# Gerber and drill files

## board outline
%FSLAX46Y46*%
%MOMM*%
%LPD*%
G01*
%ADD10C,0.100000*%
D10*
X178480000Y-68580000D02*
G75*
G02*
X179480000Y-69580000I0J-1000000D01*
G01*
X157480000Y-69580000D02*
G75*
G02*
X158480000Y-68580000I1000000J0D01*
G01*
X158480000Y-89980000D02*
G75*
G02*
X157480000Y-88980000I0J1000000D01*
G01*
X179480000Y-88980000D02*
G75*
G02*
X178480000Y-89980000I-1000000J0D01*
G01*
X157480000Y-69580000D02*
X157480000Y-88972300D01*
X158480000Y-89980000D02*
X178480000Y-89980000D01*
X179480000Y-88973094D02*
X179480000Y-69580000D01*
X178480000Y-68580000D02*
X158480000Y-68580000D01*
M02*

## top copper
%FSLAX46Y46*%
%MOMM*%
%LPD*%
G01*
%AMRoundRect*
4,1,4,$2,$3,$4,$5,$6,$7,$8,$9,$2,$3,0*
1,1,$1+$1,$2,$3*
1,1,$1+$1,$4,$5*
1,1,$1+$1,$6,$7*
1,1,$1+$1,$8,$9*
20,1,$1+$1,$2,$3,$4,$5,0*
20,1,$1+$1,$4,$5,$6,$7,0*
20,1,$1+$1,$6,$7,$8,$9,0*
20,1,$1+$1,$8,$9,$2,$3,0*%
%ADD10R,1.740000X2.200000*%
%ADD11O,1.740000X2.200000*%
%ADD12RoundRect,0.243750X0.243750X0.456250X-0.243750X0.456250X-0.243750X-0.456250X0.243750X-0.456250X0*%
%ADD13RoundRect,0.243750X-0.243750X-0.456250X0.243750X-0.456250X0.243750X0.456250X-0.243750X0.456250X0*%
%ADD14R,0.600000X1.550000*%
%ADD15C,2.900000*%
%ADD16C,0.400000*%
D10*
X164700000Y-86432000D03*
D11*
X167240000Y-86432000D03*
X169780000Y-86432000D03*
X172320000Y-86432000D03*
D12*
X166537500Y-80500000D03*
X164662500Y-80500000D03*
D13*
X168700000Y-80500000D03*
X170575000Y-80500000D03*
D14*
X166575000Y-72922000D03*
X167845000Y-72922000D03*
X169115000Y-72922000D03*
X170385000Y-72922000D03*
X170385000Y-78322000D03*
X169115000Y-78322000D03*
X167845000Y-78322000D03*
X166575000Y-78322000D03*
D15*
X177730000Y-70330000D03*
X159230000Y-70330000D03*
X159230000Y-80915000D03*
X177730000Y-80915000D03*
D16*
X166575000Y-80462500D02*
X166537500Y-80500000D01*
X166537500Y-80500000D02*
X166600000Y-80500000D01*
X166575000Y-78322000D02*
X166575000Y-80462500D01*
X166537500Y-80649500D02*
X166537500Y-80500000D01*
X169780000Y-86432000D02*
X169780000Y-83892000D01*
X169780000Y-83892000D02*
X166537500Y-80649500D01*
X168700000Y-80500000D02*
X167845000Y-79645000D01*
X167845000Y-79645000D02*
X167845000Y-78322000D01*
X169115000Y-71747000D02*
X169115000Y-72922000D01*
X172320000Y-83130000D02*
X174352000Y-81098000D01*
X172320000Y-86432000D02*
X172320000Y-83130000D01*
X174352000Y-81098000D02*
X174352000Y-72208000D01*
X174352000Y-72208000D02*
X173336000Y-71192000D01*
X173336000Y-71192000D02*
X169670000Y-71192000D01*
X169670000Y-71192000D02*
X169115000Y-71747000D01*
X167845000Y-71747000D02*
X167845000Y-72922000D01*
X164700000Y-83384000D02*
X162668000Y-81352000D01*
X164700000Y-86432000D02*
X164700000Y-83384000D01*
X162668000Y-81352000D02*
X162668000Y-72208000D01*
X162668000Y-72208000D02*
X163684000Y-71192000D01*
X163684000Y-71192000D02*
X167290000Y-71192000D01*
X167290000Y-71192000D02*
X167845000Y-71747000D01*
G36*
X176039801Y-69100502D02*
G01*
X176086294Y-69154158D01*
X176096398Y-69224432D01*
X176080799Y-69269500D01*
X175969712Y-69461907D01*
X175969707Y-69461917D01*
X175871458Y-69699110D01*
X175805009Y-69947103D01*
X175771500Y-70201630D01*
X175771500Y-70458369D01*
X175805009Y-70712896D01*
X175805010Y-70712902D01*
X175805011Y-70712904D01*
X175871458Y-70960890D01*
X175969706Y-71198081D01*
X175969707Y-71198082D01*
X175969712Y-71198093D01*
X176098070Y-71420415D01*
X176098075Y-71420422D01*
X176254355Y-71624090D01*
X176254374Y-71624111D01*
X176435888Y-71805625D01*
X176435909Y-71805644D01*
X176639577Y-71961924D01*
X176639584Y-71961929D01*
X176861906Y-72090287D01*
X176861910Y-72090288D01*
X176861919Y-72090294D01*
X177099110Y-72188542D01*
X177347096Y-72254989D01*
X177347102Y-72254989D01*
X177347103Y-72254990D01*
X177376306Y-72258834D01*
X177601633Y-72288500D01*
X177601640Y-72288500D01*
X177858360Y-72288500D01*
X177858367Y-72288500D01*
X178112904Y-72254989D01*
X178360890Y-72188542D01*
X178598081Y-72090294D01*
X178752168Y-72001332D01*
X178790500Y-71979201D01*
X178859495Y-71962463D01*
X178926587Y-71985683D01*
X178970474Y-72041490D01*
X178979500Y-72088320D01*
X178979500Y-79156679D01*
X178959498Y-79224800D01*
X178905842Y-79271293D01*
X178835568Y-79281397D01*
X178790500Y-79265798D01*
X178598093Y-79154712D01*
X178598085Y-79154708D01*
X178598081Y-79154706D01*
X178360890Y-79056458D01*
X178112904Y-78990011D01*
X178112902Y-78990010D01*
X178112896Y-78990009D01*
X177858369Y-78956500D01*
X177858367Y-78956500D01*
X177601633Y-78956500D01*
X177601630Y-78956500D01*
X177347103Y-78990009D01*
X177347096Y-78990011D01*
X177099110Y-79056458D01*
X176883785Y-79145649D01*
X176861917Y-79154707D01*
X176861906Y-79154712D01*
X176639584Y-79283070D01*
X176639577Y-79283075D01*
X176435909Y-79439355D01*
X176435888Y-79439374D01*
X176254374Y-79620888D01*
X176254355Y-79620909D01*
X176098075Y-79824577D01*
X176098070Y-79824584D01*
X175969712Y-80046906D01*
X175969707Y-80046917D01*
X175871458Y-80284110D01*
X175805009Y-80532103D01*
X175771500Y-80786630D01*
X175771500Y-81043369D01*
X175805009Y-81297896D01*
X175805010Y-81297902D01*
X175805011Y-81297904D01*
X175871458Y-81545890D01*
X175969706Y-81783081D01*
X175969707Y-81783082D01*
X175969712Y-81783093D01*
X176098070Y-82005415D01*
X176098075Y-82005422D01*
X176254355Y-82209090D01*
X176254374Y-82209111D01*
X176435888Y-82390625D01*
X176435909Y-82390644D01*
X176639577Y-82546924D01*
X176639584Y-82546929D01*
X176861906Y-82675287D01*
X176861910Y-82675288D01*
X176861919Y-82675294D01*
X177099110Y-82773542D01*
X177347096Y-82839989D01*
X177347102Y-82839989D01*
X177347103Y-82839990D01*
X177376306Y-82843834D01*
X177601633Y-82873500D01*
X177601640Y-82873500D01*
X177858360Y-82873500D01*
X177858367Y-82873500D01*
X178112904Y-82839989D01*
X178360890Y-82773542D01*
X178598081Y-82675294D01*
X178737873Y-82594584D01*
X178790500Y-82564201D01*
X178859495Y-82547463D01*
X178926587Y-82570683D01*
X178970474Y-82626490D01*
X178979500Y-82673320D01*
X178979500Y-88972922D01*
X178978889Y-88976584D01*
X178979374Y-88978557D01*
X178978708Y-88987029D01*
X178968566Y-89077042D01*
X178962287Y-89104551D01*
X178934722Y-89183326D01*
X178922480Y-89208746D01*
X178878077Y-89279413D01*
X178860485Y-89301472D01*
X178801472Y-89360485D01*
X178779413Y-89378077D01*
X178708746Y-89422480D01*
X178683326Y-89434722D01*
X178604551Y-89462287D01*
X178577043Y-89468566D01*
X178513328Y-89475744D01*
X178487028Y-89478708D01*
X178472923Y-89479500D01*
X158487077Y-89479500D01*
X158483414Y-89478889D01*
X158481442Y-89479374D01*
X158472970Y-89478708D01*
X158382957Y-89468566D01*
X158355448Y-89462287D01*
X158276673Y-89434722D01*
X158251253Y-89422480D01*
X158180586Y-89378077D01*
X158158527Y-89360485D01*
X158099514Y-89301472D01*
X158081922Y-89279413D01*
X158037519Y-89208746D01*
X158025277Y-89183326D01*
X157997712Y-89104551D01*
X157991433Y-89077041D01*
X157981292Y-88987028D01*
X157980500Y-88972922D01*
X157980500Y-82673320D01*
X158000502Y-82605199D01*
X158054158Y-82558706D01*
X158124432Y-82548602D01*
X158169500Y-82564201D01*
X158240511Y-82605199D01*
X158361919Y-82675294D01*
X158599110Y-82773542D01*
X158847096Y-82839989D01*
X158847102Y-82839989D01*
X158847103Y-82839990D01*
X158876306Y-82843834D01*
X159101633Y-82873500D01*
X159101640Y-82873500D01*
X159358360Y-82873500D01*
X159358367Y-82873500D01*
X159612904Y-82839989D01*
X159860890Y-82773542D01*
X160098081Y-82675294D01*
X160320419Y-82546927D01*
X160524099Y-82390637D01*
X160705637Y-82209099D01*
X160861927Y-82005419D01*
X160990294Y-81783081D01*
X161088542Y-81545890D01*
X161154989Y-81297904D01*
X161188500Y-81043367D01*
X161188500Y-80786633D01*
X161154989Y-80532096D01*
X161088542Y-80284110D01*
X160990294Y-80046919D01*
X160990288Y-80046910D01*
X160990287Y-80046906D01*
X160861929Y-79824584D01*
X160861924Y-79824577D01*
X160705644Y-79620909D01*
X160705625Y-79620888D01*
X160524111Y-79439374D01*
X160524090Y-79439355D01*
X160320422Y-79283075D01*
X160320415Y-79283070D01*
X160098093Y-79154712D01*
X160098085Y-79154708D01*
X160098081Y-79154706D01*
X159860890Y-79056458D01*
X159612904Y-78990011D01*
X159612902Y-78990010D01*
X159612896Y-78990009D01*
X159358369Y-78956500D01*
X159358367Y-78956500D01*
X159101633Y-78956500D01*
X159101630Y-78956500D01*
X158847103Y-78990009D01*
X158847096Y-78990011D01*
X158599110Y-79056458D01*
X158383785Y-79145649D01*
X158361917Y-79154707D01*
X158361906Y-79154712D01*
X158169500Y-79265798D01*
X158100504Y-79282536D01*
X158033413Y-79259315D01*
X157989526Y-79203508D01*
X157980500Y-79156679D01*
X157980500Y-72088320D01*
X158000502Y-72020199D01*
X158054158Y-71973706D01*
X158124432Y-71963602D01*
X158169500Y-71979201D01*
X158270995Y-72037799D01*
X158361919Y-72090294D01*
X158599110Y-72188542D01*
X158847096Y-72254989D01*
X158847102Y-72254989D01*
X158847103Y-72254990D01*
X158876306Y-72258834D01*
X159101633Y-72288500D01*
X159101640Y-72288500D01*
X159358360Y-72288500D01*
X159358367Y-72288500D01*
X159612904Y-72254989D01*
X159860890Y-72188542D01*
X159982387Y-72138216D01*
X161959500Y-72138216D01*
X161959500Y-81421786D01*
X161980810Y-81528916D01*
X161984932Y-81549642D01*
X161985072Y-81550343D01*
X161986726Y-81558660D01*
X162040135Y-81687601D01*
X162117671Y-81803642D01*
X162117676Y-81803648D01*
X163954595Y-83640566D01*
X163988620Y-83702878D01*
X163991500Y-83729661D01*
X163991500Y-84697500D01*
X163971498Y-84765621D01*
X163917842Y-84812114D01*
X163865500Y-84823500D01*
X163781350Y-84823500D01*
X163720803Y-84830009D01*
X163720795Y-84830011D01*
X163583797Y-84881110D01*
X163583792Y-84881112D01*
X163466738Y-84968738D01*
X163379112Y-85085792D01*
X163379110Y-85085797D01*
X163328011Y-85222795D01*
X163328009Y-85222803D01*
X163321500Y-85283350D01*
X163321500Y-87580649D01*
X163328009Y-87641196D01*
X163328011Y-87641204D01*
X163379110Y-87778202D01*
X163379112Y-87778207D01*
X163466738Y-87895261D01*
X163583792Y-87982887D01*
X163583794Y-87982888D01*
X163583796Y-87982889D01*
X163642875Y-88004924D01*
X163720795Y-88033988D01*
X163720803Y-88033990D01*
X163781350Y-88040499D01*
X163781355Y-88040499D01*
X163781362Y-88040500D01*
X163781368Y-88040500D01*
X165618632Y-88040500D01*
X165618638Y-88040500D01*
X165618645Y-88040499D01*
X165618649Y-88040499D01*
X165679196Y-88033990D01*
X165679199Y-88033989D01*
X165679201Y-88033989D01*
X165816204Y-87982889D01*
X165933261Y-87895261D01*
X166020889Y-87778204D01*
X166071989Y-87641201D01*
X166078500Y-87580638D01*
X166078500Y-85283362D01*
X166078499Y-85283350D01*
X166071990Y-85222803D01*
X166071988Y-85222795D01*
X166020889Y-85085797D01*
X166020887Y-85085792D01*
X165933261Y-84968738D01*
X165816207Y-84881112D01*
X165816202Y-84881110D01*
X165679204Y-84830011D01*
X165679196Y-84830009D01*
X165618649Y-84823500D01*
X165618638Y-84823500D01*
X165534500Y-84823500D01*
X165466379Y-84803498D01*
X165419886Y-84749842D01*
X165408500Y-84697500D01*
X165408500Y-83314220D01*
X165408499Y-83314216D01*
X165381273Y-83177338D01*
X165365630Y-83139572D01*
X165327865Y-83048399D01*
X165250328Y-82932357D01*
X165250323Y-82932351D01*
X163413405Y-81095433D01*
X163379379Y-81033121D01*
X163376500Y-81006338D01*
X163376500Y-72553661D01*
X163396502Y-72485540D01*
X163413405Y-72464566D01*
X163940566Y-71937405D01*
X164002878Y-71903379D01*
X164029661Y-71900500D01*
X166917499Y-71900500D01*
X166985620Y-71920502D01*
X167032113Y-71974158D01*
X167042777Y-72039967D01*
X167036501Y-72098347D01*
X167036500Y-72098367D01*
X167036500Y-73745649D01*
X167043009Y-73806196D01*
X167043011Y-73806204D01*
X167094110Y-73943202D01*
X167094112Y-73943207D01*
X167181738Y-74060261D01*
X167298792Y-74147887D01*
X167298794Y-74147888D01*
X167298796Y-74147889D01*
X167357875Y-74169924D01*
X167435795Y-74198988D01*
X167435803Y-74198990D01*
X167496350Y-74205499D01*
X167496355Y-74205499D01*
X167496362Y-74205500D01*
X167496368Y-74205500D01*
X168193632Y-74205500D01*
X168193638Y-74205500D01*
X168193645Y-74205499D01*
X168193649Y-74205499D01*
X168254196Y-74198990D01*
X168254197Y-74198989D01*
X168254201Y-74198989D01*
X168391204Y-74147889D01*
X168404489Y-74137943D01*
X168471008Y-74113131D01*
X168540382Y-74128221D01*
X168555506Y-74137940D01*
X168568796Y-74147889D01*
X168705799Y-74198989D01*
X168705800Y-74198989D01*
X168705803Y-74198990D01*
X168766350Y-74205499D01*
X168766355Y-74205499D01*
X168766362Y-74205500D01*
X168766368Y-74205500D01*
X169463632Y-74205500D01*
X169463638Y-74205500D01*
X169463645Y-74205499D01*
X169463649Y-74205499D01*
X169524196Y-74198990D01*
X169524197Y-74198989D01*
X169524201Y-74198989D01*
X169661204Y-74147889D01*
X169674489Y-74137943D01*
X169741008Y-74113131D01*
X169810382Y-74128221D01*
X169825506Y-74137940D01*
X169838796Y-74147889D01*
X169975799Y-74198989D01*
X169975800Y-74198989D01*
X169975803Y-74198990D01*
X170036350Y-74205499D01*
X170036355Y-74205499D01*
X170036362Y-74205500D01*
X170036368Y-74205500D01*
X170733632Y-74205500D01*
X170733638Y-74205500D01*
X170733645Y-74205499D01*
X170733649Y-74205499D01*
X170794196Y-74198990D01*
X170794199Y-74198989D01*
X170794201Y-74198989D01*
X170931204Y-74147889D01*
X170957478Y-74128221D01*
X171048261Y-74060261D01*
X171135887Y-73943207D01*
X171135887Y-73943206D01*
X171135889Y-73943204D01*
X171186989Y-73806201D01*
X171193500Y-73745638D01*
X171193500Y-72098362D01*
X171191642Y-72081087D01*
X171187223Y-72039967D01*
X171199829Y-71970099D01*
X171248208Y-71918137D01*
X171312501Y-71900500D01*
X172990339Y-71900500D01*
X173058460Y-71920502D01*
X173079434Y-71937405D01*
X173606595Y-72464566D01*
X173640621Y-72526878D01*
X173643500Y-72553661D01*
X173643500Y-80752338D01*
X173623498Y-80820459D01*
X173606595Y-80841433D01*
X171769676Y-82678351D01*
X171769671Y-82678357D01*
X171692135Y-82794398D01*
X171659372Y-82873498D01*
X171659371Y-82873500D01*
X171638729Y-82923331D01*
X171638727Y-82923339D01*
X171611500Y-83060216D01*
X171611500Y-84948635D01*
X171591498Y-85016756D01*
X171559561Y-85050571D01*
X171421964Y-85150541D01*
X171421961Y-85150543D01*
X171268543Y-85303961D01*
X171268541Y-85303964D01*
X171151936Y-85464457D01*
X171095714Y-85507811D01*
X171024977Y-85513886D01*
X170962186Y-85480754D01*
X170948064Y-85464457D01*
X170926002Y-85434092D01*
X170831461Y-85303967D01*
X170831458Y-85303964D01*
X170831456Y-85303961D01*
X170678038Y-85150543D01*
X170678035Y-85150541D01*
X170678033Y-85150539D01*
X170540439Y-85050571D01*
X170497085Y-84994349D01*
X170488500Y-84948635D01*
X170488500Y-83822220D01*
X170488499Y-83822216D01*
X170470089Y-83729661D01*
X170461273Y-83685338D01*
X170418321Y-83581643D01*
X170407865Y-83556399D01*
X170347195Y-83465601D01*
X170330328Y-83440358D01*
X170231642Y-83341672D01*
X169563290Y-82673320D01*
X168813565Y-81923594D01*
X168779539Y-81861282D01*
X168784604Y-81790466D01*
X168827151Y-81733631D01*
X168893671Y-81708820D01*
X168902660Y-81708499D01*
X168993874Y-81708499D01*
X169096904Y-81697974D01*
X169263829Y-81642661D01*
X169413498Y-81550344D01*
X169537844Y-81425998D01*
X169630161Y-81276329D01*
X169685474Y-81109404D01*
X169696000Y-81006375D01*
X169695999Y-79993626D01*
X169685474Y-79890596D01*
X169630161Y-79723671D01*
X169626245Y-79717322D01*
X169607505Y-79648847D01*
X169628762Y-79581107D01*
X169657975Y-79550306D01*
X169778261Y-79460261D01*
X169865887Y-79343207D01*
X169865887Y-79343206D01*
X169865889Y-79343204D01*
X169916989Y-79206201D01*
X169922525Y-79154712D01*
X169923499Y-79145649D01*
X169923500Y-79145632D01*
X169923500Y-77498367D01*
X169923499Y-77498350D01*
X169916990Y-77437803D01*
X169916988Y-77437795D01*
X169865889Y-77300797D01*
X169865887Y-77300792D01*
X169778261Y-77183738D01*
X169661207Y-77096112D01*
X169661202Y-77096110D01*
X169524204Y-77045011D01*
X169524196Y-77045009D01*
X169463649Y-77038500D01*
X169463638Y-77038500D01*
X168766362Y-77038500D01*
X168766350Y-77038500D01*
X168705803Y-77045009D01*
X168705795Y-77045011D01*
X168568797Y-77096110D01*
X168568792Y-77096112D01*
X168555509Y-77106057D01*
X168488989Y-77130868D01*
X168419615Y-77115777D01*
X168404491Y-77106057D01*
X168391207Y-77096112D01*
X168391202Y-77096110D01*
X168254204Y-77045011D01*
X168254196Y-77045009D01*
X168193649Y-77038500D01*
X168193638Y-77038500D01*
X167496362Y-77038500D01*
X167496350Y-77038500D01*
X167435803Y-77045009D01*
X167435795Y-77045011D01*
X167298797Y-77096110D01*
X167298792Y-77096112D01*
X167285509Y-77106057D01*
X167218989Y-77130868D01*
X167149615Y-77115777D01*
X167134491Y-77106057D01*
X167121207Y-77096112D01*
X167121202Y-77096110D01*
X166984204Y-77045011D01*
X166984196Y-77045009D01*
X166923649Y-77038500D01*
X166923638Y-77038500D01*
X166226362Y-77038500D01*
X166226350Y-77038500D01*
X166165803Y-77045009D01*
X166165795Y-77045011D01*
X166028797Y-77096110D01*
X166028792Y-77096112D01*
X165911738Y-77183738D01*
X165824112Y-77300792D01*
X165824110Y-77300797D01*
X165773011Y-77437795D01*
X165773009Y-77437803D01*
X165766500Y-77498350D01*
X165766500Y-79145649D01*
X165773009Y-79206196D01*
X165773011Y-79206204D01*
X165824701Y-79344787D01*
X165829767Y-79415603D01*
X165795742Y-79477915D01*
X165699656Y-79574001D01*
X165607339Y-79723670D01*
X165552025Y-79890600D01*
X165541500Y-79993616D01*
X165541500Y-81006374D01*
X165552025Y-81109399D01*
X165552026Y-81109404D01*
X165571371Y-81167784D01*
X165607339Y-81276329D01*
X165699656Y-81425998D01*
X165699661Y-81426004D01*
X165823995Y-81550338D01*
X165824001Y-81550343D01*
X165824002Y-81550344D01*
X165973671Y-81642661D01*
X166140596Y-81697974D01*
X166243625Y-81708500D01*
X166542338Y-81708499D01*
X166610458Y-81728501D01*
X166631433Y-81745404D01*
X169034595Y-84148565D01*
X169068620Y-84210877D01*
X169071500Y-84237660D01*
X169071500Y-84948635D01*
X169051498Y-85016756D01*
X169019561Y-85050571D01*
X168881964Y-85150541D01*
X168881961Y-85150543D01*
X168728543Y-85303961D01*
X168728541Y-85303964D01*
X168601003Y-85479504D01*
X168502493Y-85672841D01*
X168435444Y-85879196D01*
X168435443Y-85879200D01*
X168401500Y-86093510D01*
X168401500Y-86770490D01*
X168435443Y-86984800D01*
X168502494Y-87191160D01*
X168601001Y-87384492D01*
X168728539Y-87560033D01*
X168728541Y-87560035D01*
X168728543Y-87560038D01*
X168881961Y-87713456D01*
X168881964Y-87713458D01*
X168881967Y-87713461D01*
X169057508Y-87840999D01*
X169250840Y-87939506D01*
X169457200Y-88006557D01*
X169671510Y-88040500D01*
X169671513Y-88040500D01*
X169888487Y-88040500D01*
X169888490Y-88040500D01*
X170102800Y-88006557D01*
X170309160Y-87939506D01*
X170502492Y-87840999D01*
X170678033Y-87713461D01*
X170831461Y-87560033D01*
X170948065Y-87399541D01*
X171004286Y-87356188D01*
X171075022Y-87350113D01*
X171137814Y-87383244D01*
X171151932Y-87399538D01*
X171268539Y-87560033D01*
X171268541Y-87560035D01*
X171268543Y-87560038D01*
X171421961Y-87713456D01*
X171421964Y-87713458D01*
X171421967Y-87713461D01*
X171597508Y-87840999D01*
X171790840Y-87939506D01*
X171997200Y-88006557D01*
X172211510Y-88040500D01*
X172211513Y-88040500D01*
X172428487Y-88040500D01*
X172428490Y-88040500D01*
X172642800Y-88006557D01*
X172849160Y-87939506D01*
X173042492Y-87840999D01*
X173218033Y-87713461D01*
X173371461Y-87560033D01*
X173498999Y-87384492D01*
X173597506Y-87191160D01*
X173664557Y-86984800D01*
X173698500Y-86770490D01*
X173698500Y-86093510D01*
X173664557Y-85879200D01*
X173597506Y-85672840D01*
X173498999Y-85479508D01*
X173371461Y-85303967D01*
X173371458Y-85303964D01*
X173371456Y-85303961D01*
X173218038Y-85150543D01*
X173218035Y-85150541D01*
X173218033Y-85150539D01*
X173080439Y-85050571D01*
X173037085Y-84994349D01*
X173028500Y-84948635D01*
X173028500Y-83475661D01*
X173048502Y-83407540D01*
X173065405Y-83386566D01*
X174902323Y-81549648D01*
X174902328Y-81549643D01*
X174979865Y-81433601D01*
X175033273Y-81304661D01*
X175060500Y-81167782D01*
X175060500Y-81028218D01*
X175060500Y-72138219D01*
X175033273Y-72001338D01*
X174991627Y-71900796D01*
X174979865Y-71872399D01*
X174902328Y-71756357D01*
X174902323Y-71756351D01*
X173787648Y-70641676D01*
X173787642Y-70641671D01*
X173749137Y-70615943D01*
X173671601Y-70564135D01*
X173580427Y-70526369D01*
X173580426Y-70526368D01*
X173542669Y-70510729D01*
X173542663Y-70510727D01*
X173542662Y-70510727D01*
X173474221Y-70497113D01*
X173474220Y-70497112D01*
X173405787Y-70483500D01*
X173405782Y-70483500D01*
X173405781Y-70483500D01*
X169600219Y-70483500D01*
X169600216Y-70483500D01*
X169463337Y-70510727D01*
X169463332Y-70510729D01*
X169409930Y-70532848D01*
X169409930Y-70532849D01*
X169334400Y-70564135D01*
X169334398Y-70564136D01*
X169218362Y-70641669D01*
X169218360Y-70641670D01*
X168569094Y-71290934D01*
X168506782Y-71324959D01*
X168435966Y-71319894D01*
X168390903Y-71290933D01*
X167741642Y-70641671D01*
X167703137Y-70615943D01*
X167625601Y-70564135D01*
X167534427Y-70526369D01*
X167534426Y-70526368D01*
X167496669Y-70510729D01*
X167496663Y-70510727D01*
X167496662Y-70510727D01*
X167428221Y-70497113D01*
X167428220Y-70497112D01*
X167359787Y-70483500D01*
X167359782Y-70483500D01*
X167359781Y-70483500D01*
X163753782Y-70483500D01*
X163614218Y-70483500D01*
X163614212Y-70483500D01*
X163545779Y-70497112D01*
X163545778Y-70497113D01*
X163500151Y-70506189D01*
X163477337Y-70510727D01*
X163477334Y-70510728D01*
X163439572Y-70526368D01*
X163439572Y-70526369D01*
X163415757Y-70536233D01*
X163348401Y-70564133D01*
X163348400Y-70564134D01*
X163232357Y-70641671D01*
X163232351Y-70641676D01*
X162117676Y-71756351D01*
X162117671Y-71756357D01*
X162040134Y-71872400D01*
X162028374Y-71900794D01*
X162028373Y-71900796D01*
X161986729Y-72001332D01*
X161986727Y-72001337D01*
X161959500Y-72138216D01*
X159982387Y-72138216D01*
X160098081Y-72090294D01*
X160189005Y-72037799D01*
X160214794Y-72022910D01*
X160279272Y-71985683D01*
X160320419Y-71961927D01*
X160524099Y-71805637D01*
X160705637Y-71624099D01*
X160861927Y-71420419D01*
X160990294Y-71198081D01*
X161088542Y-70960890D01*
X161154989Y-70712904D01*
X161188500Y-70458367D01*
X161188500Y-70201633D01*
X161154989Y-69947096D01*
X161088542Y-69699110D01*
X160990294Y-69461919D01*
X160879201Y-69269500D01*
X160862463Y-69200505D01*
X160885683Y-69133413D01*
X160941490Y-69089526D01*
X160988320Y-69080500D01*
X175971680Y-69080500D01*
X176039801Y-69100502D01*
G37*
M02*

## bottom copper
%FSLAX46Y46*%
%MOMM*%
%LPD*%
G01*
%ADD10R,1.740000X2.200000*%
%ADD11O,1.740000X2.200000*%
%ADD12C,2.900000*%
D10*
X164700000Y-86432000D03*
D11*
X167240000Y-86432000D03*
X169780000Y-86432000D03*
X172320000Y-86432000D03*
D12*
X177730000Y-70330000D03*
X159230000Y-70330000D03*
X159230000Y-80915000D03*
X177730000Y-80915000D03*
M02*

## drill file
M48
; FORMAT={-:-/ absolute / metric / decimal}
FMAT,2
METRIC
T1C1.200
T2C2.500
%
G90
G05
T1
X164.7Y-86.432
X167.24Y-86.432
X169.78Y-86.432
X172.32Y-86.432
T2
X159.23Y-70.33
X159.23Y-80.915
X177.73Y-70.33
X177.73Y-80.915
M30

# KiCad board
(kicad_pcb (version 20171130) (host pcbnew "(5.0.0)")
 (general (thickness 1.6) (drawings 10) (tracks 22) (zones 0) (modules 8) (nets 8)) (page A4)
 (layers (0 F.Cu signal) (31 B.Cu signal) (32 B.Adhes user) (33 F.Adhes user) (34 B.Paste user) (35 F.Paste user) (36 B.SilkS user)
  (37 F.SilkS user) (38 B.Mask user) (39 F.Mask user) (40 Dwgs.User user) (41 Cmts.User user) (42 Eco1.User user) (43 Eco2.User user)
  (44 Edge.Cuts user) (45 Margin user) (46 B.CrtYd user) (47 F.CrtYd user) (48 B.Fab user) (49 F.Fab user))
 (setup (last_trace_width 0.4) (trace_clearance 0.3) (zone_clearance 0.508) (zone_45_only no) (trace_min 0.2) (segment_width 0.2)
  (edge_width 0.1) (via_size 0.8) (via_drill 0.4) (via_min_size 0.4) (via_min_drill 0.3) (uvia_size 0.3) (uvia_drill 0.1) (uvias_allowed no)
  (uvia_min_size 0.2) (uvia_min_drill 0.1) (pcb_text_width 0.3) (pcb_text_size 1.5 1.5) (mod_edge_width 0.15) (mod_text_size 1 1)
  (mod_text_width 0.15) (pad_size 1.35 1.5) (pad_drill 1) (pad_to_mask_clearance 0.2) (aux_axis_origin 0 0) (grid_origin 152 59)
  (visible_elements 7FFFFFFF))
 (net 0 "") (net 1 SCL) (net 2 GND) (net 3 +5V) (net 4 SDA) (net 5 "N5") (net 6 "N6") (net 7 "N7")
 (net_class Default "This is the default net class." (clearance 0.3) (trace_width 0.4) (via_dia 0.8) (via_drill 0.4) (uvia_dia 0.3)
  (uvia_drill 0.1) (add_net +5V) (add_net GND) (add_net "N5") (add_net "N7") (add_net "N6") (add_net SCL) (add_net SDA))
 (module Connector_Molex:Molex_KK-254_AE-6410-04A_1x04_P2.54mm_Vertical (layer F.Cu) (at 164.7 86.432)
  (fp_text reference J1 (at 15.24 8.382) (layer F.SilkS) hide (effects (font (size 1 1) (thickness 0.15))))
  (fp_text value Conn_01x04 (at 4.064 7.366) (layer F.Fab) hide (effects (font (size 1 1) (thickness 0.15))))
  (pad 1 thru_hole rect (at 0 0) (size 1.74 2.2) (drill 1.2) (layers *.Cu *.Mask) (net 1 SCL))
  (pad 2 thru_hole oval (at 2.54 0) (size 1.74 2.2) (drill 1.2) (layers *.Cu *.Mask) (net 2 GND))
  (pad 3 thru_hole oval (at 5.08 0) (size 1.74 2.2) (drill 1.2) (layers *.Cu *.Mask) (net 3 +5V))
  (pad 4 thru_hole oval (at 7.62 0) (size 1.74 2.2) (drill 1.2) (layers *.Cu *.Mask) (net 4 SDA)))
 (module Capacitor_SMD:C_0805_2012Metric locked (layer F.Cu) (at 165.6 80.5 180)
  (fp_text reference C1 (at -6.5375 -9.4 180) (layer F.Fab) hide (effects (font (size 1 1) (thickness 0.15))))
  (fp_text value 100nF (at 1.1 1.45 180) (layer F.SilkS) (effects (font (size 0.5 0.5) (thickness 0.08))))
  (pad 1 smd roundrect (at -0.9375 0 180) (size 0.975 1.4) (layers F.Cu F.Paste F.Mask) (roundrect_rratio 0.25) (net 3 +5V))
  (pad 2 smd roundrect (at 0.9375 0 180) (size 0.975 1.4) (layers F.Cu F.Paste F.Mask) (roundrect_rratio 0.25) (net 2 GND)))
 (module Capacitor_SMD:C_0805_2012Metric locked (layer F.Cu) (at 169.6375 80.5)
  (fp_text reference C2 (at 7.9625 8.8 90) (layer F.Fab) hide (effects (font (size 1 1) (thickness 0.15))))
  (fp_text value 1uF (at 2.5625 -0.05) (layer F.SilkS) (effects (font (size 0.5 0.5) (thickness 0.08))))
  (pad 1 smd roundrect (at -0.9375 0) (size 0.975 1.4) (layers F.Cu F.Paste F.Mask) (roundrect_rratio 0.25) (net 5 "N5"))
  (pad 2 smd roundrect (at 0.9375 0) (size 0.975 1.4) (layers F.Cu F.Paste F.Mask) (roundrect_rratio 0.25) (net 2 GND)))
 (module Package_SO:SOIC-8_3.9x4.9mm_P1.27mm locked (layer F.Cu) (at 168.48 75.622 90)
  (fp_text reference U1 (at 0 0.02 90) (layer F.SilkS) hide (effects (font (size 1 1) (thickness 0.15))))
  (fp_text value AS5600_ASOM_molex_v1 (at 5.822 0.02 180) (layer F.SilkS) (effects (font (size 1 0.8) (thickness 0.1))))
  (pad 8 smd rect (at 2.7 -1.905 90) (size 1.55 0.6) (layers F.Cu F.Paste F.Mask) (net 2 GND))
  (pad 7 smd rect (at 2.7 -0.635 90) (size 1.55 0.6) (layers F.Cu F.Paste F.Mask) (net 1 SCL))
  (pad 6 smd rect (at 2.7 0.635 90) (size 1.55 0.6) (layers F.Cu F.Paste F.Mask) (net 4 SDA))
  (pad 5 smd rect (at 2.7 1.905 90) (size 1.55 0.6) (layers F.Cu F.Paste F.Mask) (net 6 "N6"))
  (pad 4 smd rect (at -2.7 1.905 90) (size 1.55 0.6) (layers F.Cu F.Paste F.Mask) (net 2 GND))
  (pad 3 smd rect (at -2.7 0.635 90) (size 1.55 0.6) (layers F.Cu F.Paste F.Mask) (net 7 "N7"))
  (pad 2 smd rect (at -2.7 -0.635 90) (size 1.55 0.6) (layers F.Cu F.Paste F.Mask) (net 5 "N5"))
  (pad 1 smd rect (at -2.7 -1.905 90) (size 1.55 0.6) (layers F.Cu F.Paste F.Mask) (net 3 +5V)))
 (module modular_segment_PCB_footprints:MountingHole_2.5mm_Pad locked (layer F.Cu) (at 177.73 70.33)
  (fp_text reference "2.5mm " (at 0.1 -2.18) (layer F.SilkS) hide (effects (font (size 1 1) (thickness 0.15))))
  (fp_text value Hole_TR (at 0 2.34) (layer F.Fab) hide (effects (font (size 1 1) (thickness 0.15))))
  (pad "" np_thru_hole circle (at 0 0) (size 2.9 2.9) (drill 2.5) (layers *.Cu *.Mask)))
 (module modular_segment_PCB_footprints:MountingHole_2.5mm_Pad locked (layer F.Cu) (at 159.23 70.33)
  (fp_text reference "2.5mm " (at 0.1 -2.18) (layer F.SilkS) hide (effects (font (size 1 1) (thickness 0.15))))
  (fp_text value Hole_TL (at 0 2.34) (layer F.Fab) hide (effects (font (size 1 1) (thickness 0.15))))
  (pad "" np_thru_hole circle (at 0 0) (size 2.9 2.9) (drill 2.5) (layers *.Cu *.Mask)))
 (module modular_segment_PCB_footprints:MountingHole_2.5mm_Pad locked (layer F.Cu) (at 159.23 80.915)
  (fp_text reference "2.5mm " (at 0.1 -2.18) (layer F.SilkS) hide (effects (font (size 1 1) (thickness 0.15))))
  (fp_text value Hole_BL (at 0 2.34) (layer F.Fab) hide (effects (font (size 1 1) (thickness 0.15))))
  (pad "" np_thru_hole circle (at 0 0) (size 2.9 2.9) (drill 2.5) (layers *.Cu *.Mask)))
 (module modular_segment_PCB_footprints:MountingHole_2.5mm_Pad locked (layer F.Cu) (at 177.73 80.915)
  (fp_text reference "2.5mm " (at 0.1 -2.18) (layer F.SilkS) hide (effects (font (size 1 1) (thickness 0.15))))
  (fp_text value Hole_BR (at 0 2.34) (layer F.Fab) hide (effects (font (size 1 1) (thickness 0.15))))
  (pad "" np_thru_hole circle (at 0 0) (size 2.9 2.9) (drill 2.5) (layers *.Cu *.Mask)))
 (gr_arc (start 178.48 69.58) (end 179.48 69.58) (angle -90) (layer Edge.Cuts) (width 0.1))
 (gr_arc (start 158.48 69.58) (end 158.48 68.58) (angle -90) (layer Edge.Cuts) (width 0.1))
 (gr_arc (start 158.48 88.98) (end 157.48 88.98) (angle -90) (layer Edge.Cuts) (width 0.1))
 (gr_arc (start 178.48 88.98) (end 178.48 89.98) (angle -90) (layer Edge.Cuts) (width 0.1))
 (gr_line (start 157.48 69.58) (end 157.48 88.9723) (layer Edge.Cuts) (width 0.1))
 (gr_line (start 158.48 89.98) (end 178.48 89.98) (layer Edge.Cuts) (width 0.1))
 (gr_line (start 179.48 88.973094) (end 179.48 69.58) (layer Edge.Cuts) (width 0.1))
 (gr_line (start 178.48 68.58) (end 158.48 68.58) (layer Edge.Cuts) (width 0.1))
 (segment (start 166.575 80.4625) (end 166.5375 80.5) (width 0.4) (layer F.Cu) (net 3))
 (segment (start 166.5375 80.5) (end 166.6 80.5) (width 0.4) (layer F.Cu) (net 3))
 (segment (start 166.575 78.322) (end 166.575 80.4625) (width 0.4) (layer F.Cu) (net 3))
 (segment (start 166.5375 80.6495) (end 166.5375 80.5) (width 0.4) (layer F.Cu) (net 3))
 (segment (start 169.78 86.432) (end 169.78 83.892) (width 0.4) (layer F.Cu) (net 3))
 (segment (start 169.78 83.892) (end 166.5375 80.6495) (width 0.4) (layer F.Cu) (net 3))
 (segment (start 168.7 80.5) (end 167.845 79.645) (width 0.4) (layer F.Cu) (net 5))
 (segment (start 167.845 79.645) (end 167.845 78.322) (width 0.4) (layer F.Cu) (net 5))
 (segment (start 169.115 71.747) (end 169.115 72.922) (width 0.4) (layer F.Cu) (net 4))
 (segment (start 172.32 83.13) (end 174.352 81.098) (width 0.4) (layer F.Cu) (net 4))
 (segment (start 172.32 86.432) (end 172.32 83.13) (width 0.4) (layer F.Cu) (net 4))
 (segment (start 174.352 81.098) (end 174.352 72.208) (width 0.4) (layer F.Cu) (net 4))
 (segment (start 174.352 72.208) (end 173.336 71.192) (width 0.4) (layer F.Cu) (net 4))
 (segment (start 173.336 71.192) (end 169.67 71.192) (width 0.4) (layer F.Cu) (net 4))
 (segment (start 169.67 71.192) (end 169.115 71.747) (width 0.4) (layer F.Cu) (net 4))
 (segment (start 167.845 71.747) (end 167.845 72.922) (width 0.4) (layer F.Cu) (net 1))
 (segment (start 164.7 83.384) (end 162.668 81.352) (width 0.4) (layer F.Cu) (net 1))
 (segment (start 164.7 86.432) (end 164.7 83.384) (width 0.4) (layer F.Cu) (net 1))
 (segment (start 162.668 81.352) (end 162.668 72.208) (width 0.4) (layer F.Cu) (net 1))
 (segment (start 162.668 72.208) (end 163.684 71.192) (width 0.4) (layer F.Cu) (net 1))
 (segment (start 163.684 71.192) (end 167.29 71.192) (width 0.4) (layer F.Cu) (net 1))
 (segment (start 167.29 71.192) (end 167.845 71.747) (width 0.4) (layer F.Cu) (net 1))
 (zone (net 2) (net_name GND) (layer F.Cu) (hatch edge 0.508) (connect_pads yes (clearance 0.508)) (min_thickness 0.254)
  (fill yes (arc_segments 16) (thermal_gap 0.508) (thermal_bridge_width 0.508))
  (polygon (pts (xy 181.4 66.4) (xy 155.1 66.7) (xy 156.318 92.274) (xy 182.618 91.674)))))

